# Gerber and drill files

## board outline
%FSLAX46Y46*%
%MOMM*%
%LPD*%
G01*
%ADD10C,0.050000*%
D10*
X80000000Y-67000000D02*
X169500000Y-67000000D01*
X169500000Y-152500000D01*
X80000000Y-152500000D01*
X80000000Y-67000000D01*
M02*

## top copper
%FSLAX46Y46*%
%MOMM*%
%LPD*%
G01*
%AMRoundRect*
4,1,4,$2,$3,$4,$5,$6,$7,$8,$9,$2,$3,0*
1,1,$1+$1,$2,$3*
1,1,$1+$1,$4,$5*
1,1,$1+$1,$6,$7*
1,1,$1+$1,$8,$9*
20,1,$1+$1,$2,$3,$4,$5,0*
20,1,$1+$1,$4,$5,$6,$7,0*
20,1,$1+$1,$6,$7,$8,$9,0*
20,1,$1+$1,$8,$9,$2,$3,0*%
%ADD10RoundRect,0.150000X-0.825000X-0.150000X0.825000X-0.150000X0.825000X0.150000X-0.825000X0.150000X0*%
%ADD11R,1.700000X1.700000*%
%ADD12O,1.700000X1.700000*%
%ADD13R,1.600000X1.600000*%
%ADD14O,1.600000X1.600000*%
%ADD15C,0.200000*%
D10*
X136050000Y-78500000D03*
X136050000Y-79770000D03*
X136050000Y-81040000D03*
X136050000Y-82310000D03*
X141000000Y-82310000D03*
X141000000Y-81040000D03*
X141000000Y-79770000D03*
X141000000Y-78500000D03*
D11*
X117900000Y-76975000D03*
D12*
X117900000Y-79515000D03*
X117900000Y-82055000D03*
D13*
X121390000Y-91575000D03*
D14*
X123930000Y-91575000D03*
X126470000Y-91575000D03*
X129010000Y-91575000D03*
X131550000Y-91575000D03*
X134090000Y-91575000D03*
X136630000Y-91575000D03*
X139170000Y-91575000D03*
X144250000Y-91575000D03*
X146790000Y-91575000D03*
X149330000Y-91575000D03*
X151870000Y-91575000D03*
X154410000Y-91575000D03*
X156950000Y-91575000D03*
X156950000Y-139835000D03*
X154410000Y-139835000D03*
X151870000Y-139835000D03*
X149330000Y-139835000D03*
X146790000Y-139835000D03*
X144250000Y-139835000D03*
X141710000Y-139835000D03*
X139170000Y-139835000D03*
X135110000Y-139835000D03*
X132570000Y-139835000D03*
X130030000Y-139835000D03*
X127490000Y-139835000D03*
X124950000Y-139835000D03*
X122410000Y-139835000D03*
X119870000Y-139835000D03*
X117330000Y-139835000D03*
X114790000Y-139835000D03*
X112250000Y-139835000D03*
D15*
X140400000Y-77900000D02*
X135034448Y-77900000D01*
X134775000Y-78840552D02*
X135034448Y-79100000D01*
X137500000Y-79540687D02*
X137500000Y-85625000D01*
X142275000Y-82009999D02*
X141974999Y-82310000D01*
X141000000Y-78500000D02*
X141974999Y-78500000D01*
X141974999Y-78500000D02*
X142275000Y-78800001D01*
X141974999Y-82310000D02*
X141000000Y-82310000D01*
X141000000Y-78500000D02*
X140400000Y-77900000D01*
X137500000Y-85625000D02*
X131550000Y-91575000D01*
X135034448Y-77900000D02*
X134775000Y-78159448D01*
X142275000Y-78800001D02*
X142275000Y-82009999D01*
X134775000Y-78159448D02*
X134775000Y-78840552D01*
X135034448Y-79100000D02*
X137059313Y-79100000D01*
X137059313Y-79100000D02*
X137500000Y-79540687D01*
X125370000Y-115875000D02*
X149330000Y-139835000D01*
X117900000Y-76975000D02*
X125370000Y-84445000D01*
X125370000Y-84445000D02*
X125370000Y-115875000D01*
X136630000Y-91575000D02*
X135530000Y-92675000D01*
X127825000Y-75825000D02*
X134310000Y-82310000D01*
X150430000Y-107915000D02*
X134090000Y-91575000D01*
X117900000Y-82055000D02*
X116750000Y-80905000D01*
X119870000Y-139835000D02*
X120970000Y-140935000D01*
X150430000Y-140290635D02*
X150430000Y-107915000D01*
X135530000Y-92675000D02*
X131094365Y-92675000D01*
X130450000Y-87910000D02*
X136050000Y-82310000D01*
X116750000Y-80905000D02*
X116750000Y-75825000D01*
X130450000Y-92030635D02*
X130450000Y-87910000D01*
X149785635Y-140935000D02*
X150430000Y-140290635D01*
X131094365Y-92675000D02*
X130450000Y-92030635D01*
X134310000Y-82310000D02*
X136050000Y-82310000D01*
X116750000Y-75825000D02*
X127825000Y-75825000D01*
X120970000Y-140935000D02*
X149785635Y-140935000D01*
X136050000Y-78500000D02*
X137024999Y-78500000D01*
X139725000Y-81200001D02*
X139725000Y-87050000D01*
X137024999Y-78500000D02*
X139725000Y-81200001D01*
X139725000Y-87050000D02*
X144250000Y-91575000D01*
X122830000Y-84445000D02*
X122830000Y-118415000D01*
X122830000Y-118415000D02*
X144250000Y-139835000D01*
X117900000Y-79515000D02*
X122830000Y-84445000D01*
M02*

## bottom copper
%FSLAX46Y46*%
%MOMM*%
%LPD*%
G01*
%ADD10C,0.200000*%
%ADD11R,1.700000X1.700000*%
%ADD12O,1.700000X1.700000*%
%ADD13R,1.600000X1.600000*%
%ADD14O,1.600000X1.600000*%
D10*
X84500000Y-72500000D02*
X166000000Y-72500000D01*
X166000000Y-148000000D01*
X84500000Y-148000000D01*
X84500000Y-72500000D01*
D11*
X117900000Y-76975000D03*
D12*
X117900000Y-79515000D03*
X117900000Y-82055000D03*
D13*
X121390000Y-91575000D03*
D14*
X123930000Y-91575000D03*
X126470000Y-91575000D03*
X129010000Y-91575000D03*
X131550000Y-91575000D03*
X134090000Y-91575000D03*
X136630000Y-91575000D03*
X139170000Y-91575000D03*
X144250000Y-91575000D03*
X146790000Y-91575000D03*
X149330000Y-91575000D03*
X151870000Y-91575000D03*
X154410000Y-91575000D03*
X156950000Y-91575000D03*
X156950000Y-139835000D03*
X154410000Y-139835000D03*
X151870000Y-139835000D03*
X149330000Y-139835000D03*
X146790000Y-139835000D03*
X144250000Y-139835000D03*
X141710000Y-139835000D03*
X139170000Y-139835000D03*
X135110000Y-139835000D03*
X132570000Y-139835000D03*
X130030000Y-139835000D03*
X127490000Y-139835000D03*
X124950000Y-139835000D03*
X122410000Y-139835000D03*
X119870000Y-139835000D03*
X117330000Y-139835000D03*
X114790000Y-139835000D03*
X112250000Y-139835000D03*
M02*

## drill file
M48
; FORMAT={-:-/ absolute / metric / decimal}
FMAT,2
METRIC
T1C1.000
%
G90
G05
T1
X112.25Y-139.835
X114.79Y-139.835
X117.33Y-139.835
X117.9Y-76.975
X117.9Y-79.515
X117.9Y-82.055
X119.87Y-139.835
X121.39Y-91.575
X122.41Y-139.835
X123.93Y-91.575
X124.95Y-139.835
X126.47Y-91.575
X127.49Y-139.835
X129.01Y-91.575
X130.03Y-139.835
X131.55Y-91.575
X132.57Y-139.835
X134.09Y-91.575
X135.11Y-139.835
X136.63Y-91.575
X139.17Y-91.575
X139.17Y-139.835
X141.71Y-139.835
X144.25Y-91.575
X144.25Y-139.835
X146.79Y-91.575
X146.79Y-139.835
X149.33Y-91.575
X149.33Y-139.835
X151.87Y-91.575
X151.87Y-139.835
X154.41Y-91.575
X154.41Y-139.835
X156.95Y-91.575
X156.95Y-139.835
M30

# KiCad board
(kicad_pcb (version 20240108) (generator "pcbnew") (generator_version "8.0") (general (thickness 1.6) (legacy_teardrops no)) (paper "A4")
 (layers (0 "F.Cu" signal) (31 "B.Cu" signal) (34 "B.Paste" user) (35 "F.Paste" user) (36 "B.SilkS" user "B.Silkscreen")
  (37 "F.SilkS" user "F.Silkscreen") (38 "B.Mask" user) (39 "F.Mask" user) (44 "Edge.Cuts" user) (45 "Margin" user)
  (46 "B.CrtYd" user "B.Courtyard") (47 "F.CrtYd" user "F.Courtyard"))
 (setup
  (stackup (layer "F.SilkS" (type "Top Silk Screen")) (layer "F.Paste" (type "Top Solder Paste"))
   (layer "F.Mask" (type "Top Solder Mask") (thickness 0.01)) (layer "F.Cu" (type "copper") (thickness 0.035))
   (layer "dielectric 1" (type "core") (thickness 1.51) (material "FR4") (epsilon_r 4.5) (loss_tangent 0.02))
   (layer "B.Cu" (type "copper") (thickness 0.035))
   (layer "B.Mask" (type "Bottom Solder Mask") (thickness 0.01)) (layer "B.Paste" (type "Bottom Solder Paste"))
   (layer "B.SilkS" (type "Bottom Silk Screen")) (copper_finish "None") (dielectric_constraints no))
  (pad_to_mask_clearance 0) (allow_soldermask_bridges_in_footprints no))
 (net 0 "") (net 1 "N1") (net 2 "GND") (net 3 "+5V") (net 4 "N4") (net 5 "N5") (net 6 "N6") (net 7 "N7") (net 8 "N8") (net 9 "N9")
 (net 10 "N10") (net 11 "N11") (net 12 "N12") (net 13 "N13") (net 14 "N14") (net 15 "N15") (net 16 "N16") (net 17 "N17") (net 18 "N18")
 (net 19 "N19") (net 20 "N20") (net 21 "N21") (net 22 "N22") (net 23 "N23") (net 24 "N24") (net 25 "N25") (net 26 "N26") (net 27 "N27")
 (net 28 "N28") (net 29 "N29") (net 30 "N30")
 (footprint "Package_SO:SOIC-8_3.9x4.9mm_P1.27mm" (layer "F.Cu") (at 138.525 80.405)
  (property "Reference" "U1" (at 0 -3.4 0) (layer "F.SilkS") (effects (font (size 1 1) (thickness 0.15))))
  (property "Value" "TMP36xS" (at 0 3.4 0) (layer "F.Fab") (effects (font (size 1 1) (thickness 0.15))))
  (pad "1" smd roundrect (at -2.475 -1.905) (size 1.95 0.6) (layers "F.Cu" "F.Paste" "F.Mask") (roundrect_rratio 0.25) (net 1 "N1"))
  (pad "2" smd roundrect (at -2.475 -0.635) (size 1.95 0.6) (layers "F.Cu" "F.Paste" "F.Mask") (roundrect_rratio 0.25))
  (pad "3" smd roundrect (at -2.475 0.635) (size 1.95 0.6) (layers "F.Cu" "F.Paste" "F.Mask") (roundrect_rratio 0.25))
  (pad "4" smd roundrect (at -2.475 1.905) (size 1.95 0.6) (layers "F.Cu" "F.Paste" "F.Mask") (roundrect_rratio 0.25) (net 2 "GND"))
  (pad "5" smd roundrect (at 2.475 1.905) (size 1.95 0.6) (layers "F.Cu" "F.Paste" "F.Mask") (roundrect_rratio 0.25) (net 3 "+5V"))
  (pad "6" smd roundrect (at 2.475 0.635) (size 1.95 0.6) (layers "F.Cu" "F.Paste" "F.Mask") (roundrect_rratio 0.25))
  (pad "7" smd roundrect (at 2.475 -0.635) (size 1.95 0.6) (layers "F.Cu" "F.Paste" "F.Mask") (roundrect_rratio 0.25))
  (pad "8" smd roundrect (at 2.475 -1.905) (size 1.95 0.6) (layers "F.Cu" "F.Paste" "F.Mask") (roundrect_rratio 0.25) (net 3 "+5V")))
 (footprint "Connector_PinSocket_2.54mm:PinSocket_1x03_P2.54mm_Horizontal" (layer "F.Cu") (at 117.9 76.975)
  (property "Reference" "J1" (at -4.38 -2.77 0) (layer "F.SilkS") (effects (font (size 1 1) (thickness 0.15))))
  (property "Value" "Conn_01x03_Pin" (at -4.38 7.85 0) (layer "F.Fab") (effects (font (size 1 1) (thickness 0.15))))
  (pad "1" thru_hole rect (at 0 0) (size 1.7 1.7) (drill 1) (layers "*.Cu" "*.Mask") (remove_unused_layers no) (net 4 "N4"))
  (pad "2" thru_hole oval (at 0 2.54) (size 1.7 1.7) (drill 1) (layers "*.Cu" "*.Mask") (remove_unused_layers no) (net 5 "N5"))
  (pad "3" thru_hole oval (at 0 5.08) (size 1.7 1.7) (drill 1) (layers "*.Cu" "*.Mask") (remove_unused_layers no) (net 2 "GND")))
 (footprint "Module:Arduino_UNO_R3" (layer "F.Cu") (at 121.39 91.575)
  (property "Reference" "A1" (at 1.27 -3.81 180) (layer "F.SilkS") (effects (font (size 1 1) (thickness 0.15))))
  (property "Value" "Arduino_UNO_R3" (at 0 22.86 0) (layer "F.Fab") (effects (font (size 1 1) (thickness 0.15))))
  (pad "1" thru_hole rect (at 0 0 90) (size 1.6 1.6) (drill 1) (layers "*.Cu" "*.Mask") (remove_unused_layers no) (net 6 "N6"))
  (pad "2" thru_hole oval (at 2.54 0 90) (size 1.6 1.6) (drill 1) (layers "*.Cu" "*.Mask") (remove_unused_layers no) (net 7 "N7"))
  (pad "3" thru_hole oval (at 5.08 0 90) (size 1.6 1.6) (drill 1) (layers "*.Cu" "*.Mask") (remove_unused_layers no) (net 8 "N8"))
  (pad "4" thru_hole oval (at 7.62 0 90) (size 1.6 1.6) (drill 1) (layers "*.Cu" "*.Mask") (remove_unused_layers no) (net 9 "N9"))
  (pad "5" thru_hole oval (at 10.16 0 90) (size 1.6 1.6) (drill 1) (layers "*.Cu" "*.Mask") (remove_unused_layers no) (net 3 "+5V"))
  (pad "6" thru_hole oval (at 12.7 0 90) (size 1.6 1.6) (drill 1) (layers "*.Cu" "*.Mask") (remove_unused_layers no) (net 2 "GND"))
  (pad "7" thru_hole oval (at 15.24 0 90) (size 1.6 1.6) (drill 1) (layers "*.Cu" "*.Mask") (remove_unused_layers no) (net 2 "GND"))
  (pad "8" thru_hole oval (at 17.78 0 90) (size 1.6 1.6) (drill 1) (layers "*.Cu" "*.Mask") (remove_unused_layers no) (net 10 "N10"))
  (pad "9" thru_hole oval (at 22.86 0 90) (size 1.6 1.6) (drill 1) (layers "*.Cu" "*.Mask") (remove_unused_layers no) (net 1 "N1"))
  (pad "10" thru_hole oval (at 25.4 0 90) (size 1.6 1.6) (drill 1) (layers "*.Cu" "*.Mask") (remove_unused_layers no) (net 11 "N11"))
  (pad "11" thru_hole oval (at 27.94 0 90) (size 1.6 1.6) (drill 1) (layers "*.Cu" "*.Mask") (remove_unused_layers no) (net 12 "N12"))
  (pad "12" thru_hole oval (at 30.48 0 90) (size 1.6 1.6) (drill 1) (layers "*.Cu" "*.Mask") (remove_unused_layers no) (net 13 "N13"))
  (pad "13" thru_hole oval (at 33.02 0 90) (size 1.6 1.6) (drill 1) (layers "*.Cu" "*.Mask") (remove_unused_layers no) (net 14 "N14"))
  (pad "14" thru_hole oval (at 35.56 0 90) (size 1.6 1.6) (drill 1) (layers "*.Cu" "*.Mask") (remove_unused_layers no) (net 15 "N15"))
  (pad "15" thru_hole oval (at 35.56 48.26 90) (size 1.6 1.6) (drill 1) (layers "*.Cu" "*.Mask") (remove_unused_layers no) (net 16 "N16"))
  (pad "16" thru_hole oval (at 33.02 48.26 90) (size 1.6 1.6) (drill 1) (layers "*.Cu" "*.Mask") (remove_unused_layers no) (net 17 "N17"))
  (pad "17" thru_hole oval (at 30.48 48.26 90) (size 1.6 1.6) (drill 1) (layers "*.Cu" "*.Mask") (remove_unused_layers no) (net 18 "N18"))
  (pad "18" thru_hole oval (at 27.94 48.26 90) (size 1.6 1.6) (drill 1) (layers "*.Cu" "*.Mask") (remove_unused_layers no) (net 4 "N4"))
  (pad "19" thru_hole oval (at 25.4 48.26 90) (size 1.6 1.6) (drill 1) (layers "*.Cu" "*.Mask") (remove_unused_layers no) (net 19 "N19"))
  (pad "20" thru_hole oval (at 22.86 48.26 90) (size 1.6 1.6) (drill 1) (layers "*.Cu" "*.Mask") (remove_unused_layers no) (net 5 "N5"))
  (pad "21" thru_hole oval (at 20.32 48.26 90) (size 1.6 1.6) (drill 1) (layers "*.Cu" "*.Mask") (remove_unused_layers no) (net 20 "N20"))
  (pad "22" thru_hole oval (at 17.78 48.26 90) (size 1.6 1.6) (drill 1) (layers "*.Cu" "*.Mask") (remove_unused_layers no) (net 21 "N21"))
  (pad "23" thru_hole oval (at 13.72 48.26 90) (size 1.6 1.6) (drill 1) (layers "*.Cu" "*.Mask") (remove_unused_layers no) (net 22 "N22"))
  (pad "24" thru_hole oval (at 11.18 48.26 90) (size 1.6 1.6) (drill 1) (layers "*.Cu" "*.Mask") (remove_unused_layers no) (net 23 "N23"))
  (pad "25" thru_hole oval (at 8.64 48.26 90) (size 1.6 1.6) (drill 1) (layers "*.Cu" "*.Mask") (remove_unused_layers no) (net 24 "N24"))
  (pad "26" thru_hole oval (at 6.1 48.26 90) (size 1.6 1.6) (drill 1) (layers "*.Cu" "*.Mask") (remove_unused_layers no) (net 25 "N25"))
  (pad "27" thru_hole oval (at 3.56 48.26 90) (size 1.6 1.6) (drill 1) (layers "*.Cu" "*.Mask") (remove_unused_layers no) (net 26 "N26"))
  (pad "28" thru_hole oval (at 1.02 48.26 90) (size 1.6 1.6) (drill 1) (layers "*.Cu" "*.Mask") (remove_unused_layers no) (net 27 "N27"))
  (pad "29" thru_hole oval (at -1.52 48.26 90) (size 1.6 1.6) (drill 1) (layers "*.Cu" "*.Mask") (remove_unused_layers no) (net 2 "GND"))
  (pad "30" thru_hole oval (at -4.06 48.26 90) (size 1.6 1.6) (drill 1) (layers "*.Cu" "*.Mask") (remove_unused_layers no) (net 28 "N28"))
  (pad "31" thru_hole oval (at -6.6 48.26 90) (size 1.6 1.6) (drill 1) (layers "*.Cu" "*.Mask") (remove_unused_layers no) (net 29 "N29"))
  (pad "32" thru_hole oval (at -9.14 48.26 90) (size 1.6 1.6) (drill 1) (layers "*.Cu" "*.Mask") (remove_unused_layers no) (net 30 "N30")))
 (gr_rect (start 84.5 72.5) (end 166 148) (stroke (width 0.2) (type default)) (fill none) (layer "B.Cu"))
 (gr_rect (start 80 67) (end 169.5 152.5) (stroke (width 0.05) (type default)) (fill none) (layer "Edge.Cuts"))
 (segment (start 140.4 77.9) (end 135.034448 77.9) (width 0.2) (layer "F.Cu") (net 3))
 (segment (start 134.775 78.840552) (end 135.034448 79.1) (width 0.2) (layer "F.Cu") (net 3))
 (segment (start 137.5 79.540687) (end 137.5 85.625) (width 0.2) (layer "F.Cu") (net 3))
 (segment (start 142.275 82.009999) (end 141.974999 82.31) (width 0.2) (layer "F.Cu") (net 3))
 (segment (start 141 78.5) (end 141.974999 78.5) (width 0.2) (layer "F.Cu") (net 3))
 (segment (start 141.974999 78.5) (end 142.275 78.800001) (width 0.2) (layer "F.Cu") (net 3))
 (segment (start 141.974999 82.31) (end 141 82.31) (width 0.2) (layer "F.Cu") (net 3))
 (segment (start 141 78.5) (end 140.4 77.9) (width 0.2) (layer "F.Cu") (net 3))
 (segment (start 137.5 85.625) (end 131.55 91.575) (width 0.2) (layer "F.Cu") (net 3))
 (segment (start 135.034448 77.9) (end 134.775 78.159448) (width 0.2) (layer "F.Cu") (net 3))
 (segment (start 142.275 78.800001) (end 142.275 82.009999) (width 0.2) (layer "F.Cu") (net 3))
 (segment (start 134.775 78.159448) (end 134.775 78.840552) (width 0.2) (layer "F.Cu") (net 3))
 (segment (start 135.034448 79.1) (end 137.059313 79.1) (width 0.2) (layer "F.Cu") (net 3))
 (segment (start 137.059313 79.1) (end 137.5 79.540687) (width 0.2) (layer "F.Cu") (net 3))
 (segment (start 125.37 115.875) (end 149.33 139.835) (width 0.2) (layer "F.Cu") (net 4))
 (segment (start 117.9 76.975) (end 125.37 84.445) (width 0.2) (layer "F.Cu") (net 4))
 (segment (start 125.37 84.445) (end 125.37 115.875) (width 0.2) (layer "F.Cu") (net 4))
 (segment (start 136.63 91.575) (end 135.53 92.675) (width 0.2) (layer "F.Cu") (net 2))
 (segment (start 127.825 75.825) (end 134.31 82.31) (width 0.2) (layer "F.Cu") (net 2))
 (segment (start 150.43 107.915) (end 134.09 91.575) (width 0.2) (layer "F.Cu") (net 2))
 (segment (start 117.9 82.055) (end 116.75 80.905) (width 0.2) (layer "F.Cu") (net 2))
 (segment (start 119.87 139.835) (end 120.97 140.935) (width 0.2) (layer "F.Cu") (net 2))
 (segment (start 150.43 140.290635) (end 150.43 107.915) (width 0.2) (layer "F.Cu") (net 2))
 (segment (start 135.53 92.675) (end 131.094365 92.675) (width 0.2) (layer "F.Cu") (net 2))
 (segment (start 130.45 87.91) (end 136.05 82.31) (width 0.2) (layer "F.Cu") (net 2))
 (segment (start 116.75 80.905) (end 116.75 75.825) (width 0.2) (layer "F.Cu") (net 2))
 (segment (start 130.45 92.030635) (end 130.45 87.91) (width 0.2) (layer "F.Cu") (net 2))
 (segment (start 149.785635 140.935) (end 150.43 140.290635) (width 0.2) (layer "F.Cu") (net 2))
 (segment (start 131.094365 92.675) (end 130.45 92.030635) (width 0.2) (layer "F.Cu") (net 2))
 (segment (start 134.31 82.31) (end 136.05 82.31) (width 0.2) (layer "F.Cu") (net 2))
 (segment (start 116.75 75.825) (end 127.825 75.825) (width 0.2) (layer "F.Cu") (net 2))
 (segment (start 120.97 140.935) (end 149.785635 140.935) (width 0.2) (layer "F.Cu") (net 2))
 (segment (start 136.05 78.5) (end 137.024999 78.5) (width 0.2) (layer "F.Cu") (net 1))
 (segment (start 139.725 81.200001) (end 139.725 87.05) (width 0.2) (layer "F.Cu") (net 1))
 (segment (start 137.024999 78.5) (end 139.725 81.200001) (width 0.2) (layer "F.Cu") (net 1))
 (segment (start 139.725 87.05) (end 144.25 91.575) (width 0.2) (layer "F.Cu") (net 1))
 (segment (start 122.83 84.445) (end 122.83 118.415) (width 0.2) (layer "F.Cu") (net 5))
 (segment (start 122.83 118.415) (end 144.25 139.835) (width 0.2) (layer "F.Cu") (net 5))
 (segment (start 117.9 79.515) (end 122.83 84.445) (width 0.2) (layer "F.Cu") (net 5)))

